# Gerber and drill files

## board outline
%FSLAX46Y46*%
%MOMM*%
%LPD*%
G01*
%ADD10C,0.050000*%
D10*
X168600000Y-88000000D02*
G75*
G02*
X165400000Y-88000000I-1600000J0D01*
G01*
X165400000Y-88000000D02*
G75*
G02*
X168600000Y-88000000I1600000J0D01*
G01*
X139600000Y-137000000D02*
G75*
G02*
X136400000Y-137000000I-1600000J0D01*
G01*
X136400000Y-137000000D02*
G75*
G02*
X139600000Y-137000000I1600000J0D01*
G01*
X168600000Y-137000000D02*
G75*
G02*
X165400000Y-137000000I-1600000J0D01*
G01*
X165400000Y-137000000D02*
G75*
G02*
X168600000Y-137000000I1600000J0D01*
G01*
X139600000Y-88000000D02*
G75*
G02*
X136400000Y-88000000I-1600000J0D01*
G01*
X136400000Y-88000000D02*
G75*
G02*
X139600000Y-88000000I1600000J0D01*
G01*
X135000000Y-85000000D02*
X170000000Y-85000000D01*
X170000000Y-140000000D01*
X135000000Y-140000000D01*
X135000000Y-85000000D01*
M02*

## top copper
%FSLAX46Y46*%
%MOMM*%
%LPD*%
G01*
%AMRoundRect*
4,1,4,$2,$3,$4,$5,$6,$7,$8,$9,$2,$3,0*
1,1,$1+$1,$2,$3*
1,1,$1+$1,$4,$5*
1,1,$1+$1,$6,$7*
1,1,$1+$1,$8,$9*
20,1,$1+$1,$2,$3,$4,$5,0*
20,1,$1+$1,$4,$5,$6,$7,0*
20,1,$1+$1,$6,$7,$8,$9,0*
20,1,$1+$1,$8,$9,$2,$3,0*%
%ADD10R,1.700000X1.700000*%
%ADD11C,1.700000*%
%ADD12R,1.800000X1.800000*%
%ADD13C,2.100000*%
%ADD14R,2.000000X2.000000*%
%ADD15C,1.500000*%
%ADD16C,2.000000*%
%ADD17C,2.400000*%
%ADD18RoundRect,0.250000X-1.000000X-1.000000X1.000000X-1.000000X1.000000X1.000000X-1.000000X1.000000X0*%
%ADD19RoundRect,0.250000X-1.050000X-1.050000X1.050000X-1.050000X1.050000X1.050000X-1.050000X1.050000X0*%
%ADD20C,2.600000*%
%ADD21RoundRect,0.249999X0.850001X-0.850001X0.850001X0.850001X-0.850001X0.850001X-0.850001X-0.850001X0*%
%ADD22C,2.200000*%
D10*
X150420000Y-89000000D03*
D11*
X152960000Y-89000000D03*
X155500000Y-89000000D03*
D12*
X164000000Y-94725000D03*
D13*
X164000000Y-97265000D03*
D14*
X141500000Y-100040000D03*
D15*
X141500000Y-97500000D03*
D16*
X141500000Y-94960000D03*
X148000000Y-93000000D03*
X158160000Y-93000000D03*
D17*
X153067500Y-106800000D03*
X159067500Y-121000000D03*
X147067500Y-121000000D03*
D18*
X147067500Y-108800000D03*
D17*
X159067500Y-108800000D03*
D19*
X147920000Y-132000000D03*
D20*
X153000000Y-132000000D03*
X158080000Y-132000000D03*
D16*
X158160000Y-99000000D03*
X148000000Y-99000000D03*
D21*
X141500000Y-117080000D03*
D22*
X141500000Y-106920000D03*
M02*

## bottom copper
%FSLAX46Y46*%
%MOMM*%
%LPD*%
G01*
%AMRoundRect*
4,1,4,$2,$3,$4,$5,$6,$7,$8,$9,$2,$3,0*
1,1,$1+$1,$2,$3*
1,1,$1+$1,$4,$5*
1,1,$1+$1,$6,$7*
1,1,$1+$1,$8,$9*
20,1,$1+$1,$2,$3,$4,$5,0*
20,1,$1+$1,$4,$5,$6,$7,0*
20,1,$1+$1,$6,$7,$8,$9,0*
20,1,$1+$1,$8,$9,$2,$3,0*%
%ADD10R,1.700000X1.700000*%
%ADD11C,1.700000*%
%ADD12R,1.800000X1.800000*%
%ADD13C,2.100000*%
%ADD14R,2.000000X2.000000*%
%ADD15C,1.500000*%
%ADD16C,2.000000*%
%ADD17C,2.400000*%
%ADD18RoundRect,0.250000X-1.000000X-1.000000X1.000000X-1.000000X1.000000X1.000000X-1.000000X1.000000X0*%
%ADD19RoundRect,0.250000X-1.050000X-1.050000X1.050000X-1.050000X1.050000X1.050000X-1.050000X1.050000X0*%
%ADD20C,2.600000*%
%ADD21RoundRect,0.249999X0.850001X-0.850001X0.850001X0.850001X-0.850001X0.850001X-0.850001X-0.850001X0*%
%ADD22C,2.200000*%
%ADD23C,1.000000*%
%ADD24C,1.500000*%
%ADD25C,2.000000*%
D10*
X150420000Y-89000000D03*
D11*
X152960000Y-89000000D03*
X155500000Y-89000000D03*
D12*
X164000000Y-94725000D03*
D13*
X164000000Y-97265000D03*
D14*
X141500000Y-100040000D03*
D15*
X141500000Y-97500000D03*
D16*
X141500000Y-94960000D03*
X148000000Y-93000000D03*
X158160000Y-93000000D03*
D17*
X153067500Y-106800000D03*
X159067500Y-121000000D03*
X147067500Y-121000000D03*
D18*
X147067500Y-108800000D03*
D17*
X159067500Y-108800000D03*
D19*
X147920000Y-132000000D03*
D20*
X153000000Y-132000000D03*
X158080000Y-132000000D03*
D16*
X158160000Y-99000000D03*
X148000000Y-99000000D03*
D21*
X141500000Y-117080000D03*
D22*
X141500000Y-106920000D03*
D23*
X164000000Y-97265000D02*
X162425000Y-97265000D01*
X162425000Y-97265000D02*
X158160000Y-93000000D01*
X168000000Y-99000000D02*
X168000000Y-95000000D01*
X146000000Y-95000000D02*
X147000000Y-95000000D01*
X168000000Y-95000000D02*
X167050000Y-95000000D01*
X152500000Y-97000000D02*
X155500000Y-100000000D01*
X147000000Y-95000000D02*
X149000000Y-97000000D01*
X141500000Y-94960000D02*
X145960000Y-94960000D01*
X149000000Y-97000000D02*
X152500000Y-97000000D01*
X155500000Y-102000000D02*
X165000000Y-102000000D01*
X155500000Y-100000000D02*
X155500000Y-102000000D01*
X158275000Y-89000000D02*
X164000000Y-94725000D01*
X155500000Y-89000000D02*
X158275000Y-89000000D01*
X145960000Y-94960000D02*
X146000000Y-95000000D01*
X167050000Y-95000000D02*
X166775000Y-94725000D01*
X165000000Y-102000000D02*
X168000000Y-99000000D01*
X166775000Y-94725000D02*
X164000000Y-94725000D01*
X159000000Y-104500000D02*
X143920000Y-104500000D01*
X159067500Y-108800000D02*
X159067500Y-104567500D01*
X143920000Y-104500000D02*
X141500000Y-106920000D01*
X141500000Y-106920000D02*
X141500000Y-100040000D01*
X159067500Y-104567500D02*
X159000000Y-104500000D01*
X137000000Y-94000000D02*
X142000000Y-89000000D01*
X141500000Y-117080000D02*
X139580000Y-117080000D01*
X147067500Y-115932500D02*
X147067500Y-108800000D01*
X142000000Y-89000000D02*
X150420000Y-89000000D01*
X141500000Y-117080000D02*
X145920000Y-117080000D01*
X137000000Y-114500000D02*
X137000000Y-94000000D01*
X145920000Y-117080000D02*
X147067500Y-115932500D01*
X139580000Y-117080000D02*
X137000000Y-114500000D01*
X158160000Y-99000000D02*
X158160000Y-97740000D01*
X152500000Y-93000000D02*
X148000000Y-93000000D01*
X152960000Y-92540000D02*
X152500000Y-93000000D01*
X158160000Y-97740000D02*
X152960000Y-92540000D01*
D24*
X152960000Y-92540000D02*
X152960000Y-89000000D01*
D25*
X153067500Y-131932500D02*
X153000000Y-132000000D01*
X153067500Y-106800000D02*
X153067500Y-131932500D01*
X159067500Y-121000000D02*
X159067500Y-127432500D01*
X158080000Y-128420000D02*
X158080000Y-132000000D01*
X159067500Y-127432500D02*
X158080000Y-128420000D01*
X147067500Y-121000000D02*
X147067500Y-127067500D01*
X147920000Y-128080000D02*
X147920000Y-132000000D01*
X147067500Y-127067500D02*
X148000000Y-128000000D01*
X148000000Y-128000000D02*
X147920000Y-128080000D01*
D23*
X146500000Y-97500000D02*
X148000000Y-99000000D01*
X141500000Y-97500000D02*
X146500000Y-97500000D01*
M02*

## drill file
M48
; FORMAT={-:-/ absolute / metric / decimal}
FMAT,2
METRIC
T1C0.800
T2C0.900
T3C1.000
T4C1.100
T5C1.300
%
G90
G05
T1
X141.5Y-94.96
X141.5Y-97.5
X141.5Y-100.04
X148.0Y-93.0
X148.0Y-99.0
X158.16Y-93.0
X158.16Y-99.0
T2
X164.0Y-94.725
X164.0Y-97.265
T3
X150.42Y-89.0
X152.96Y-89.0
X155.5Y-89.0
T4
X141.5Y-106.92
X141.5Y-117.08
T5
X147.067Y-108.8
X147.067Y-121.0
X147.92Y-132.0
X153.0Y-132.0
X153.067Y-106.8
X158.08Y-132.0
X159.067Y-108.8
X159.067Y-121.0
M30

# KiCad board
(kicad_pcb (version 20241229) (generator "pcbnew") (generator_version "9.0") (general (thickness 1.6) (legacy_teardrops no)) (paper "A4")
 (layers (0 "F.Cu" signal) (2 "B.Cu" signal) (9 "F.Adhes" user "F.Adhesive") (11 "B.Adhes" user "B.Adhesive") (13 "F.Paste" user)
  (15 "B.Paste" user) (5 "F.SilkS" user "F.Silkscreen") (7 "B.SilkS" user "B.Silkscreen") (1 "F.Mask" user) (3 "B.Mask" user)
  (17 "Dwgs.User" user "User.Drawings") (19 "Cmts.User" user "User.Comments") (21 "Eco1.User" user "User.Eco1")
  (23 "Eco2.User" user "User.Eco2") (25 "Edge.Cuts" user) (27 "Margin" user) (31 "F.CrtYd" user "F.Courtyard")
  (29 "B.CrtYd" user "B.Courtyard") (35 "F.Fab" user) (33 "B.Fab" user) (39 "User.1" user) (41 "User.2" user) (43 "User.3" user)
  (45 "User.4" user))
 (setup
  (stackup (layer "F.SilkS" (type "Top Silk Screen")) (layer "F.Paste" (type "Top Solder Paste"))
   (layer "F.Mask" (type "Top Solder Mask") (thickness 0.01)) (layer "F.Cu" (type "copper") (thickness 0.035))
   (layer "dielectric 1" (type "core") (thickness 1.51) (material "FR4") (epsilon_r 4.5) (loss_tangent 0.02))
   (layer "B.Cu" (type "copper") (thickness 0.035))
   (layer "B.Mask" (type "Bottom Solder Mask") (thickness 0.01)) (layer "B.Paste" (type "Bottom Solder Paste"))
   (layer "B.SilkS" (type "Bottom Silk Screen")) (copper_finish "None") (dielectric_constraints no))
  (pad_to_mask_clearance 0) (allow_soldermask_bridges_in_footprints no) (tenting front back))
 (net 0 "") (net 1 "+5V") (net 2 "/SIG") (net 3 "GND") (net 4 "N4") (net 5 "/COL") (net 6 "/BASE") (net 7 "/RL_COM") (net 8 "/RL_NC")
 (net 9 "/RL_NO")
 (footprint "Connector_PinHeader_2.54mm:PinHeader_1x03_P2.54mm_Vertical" (layer "F.Cu") (at 150.42 89 90)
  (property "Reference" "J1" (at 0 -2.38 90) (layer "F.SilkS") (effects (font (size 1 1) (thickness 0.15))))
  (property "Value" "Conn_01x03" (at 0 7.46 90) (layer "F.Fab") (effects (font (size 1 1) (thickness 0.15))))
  (pad "1" thru_hole rect (at 0 0 90) (size 1.7 1.7) (drill 1) (layers "*.Cu" "*.Mask") (remove_unused_layers no) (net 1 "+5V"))
  (pad "2" thru_hole circle (at 0 2.54 90) (size 1.7 1.7) (drill 1) (layers "*.Cu" "*.Mask") (remove_unused_layers no) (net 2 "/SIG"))
  (pad "3" thru_hole circle (at 0 5.08 90) (size 1.7 1.7) (drill 1) (layers "*.Cu" "*.Mask") (remove_unused_layers no) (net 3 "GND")))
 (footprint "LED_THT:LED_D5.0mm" (layer "F.Cu") (at 164 94.725 -90)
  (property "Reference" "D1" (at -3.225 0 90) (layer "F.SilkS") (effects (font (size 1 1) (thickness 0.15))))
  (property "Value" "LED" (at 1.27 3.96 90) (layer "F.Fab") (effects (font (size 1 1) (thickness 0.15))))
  (pad "1" thru_hole rect (at 0 0 270) (size 1.8 1.8) (drill 0.9) (layers "*.Cu" "*.Mask") (remove_unused_layers no) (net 3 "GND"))
  (pad "2" thru_hole circle (at 2.54 0 270) (size 2.1 2.1) (drill 0.9) (layers "*.Cu" "*.Mask") (remove_unused_layers no) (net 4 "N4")))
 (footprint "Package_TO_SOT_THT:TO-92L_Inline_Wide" (layer "F.Cu") (at 141.5 100.04 90)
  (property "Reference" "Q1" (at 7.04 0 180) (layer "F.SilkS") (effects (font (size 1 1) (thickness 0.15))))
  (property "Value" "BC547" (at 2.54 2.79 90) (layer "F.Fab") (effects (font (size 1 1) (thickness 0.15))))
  (pad "1" thru_hole rect (at 0 0 90) (size 2 2) (drill 0.8) (layers "*.Cu" "*.Mask") (remove_unused_layers no) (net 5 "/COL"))
  (pad "2" thru_hole circle (at 2.54 0 90) (size 1.5 1.5) (drill 0.8) (layers "*.Cu" "*.Mask") (remove_unused_layers no) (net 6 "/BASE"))
  (pad "3" thru_hole circle (at 5.08 0 90) (size 2 2) (drill 0.8) (layers "*.Cu" "*.Mask") (remove_unused_layers no) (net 3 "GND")))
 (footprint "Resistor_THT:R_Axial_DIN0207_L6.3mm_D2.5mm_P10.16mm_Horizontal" (layer "F.Cu") (at 148 93)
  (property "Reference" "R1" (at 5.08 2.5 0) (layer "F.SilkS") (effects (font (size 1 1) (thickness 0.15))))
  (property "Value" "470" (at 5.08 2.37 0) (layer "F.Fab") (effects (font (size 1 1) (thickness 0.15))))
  (pad "1" thru_hole circle (at 0 0) (size 2 2) (drill 0.8) (layers "*.Cu" "*.Mask") (remove_unused_layers no) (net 2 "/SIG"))
  (pad "2" thru_hole circle (at 10.16 0) (size 2 2) (drill 0.8) (layers "*.Cu" "*.Mask") (remove_unused_layers no) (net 4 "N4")))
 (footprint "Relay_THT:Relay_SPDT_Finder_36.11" (layer "F.Cu") (at 147.0675 108.8)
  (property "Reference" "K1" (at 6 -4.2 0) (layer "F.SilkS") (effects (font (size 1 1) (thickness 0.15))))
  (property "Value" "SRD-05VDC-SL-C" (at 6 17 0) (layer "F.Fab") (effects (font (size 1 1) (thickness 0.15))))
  (pad "11" thru_hole circle (at 6 -2) (size 2.4 2.4) (drill 1.3) (layers "*.Cu" "*.Mask") (remove_unused_layers no) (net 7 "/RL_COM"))
  (pad "12" thru_hole circle (at 12 12.2) (size 2.4 2.4) (drill 1.3) (layers "*.Cu" "*.Mask") (remove_unused_layers no) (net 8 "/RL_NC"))
  (pad "14" thru_hole circle (at 0 12.2) (size 2.4 2.4) (drill 1.3) (layers "*.Cu" "*.Mask") (remove_unused_layers no) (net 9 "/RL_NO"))
  (pad "A1" thru_hole roundrect (at 0 0) (size 2.5 2.5) (drill 1.3) (layers "*.Cu" "*.Mask") (remove_unused_layers no)
   (roundrect_rratio 0.1) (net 1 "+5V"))
  (pad "A2" thru_hole circle (at 12 0) (size 2.4 2.4) (drill 1.3) (layers "*.Cu" "*.Mask") (remove_unused_layers no) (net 5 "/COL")))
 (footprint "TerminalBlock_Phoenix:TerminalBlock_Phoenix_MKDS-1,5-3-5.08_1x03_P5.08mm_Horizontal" (layer "F.Cu") (at 147.92 132)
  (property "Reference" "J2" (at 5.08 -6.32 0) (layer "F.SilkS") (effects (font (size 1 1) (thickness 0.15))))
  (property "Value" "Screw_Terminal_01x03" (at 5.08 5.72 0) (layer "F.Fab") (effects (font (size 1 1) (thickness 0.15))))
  (pad "1" thru_hole roundrect (at 0 0) (size 2.6 2.6) (drill 1.3) (layers "*.Cu" "*.Mask") (remove_unused_layers no)
   (roundrect_rratio 0.096154) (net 9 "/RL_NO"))
  (pad "2" thru_hole circle (at 5.08 0) (size 2.6 2.6) (drill 1.3) (layers "*.Cu" "*.Mask") (remove_unused_layers no) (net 7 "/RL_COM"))
  (pad "3" thru_hole circle (at 10.16 0) (size 2.6 2.6) (drill 1.3) (layers "*.Cu" "*.Mask") (remove_unused_layers no) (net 8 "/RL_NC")))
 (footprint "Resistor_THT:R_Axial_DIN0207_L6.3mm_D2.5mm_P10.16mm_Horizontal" (layer "F.Cu") (at 158.16 99 180)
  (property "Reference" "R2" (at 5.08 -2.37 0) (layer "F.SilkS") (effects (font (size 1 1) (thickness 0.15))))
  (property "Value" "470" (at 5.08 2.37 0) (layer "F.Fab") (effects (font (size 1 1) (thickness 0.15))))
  (pad "1" thru_hole circle (at 0 0 180) (size 2 2) (drill 0.8) (layers "*.Cu" "*.Mask") (remove_unused_layers no) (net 2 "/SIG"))
  (pad "2" thru_hole circle (at 10.16 0 180) (size 2 2) (drill 0.8) (layers "*.Cu" "*.Mask") (remove_unused_layers no) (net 6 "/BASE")))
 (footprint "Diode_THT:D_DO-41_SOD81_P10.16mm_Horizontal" (layer "F.Cu") (at 141.5 117.08 90)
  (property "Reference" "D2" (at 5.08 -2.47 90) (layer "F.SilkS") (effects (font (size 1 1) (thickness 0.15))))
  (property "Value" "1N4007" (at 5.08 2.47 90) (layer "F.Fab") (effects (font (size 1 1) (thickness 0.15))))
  (pad "1" thru_hole roundrect (at 0 0 90) (size 2.2 2.2) (drill 1.1) (layers "*.Cu" "*.Mask") (remove_unused_layers no)
   (roundrect_rratio 0.113636) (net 1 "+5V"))
  (pad "2" thru_hole circle (at 10.16 0 90) (size 2.2 2.2) (drill 1.1) (layers "*.Cu" "*.Mask") (remove_unused_layers no) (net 5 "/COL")))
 (gr_circle (center 167 88) (end 168.6 88) (stroke (width 0.05) (type default)) (fill no) (locked yes) (layer "Edge.Cuts"))
 (gr_circle (center 138 137) (end 139.6 137) (stroke (width 0.05) (type default)) (fill no) (locked yes) (layer "Edge.Cuts"))
 (gr_circle (center 167 137) (end 168.6 137) (stroke (width 0.05) (type default)) (fill no) (locked yes) (layer "Edge.Cuts"))
 (gr_circle (center 138 88) (end 139.6 88) (stroke (width 0.05) (type default)) (fill no) (locked yes) (layer "Edge.Cuts"))
 (gr_rect (start 135 85) (end 170 140) (stroke (width 0.05) (type default)) (fill no) (locked yes) (layer "Edge.Cuts"))
 (segment (start 164 97.265) (end 162.425 97.265) (width 1) (layer "B.Cu") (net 4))
 (segment (start 162.425 97.265) (end 158.16 93) (width 1) (layer "B.Cu") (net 4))
 (segment (start 168 99) (end 168 95) (width 1) (layer "B.Cu") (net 3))
 (segment (start 146 95) (end 147 95) (width 1) (layer "B.Cu") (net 3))
 (segment (start 168 95) (end 167.05 95) (width 1) (layer "B.Cu") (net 3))
 (segment (start 152.5 97) (end 155.5 100) (width 1) (layer "B.Cu") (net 3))
 (segment (start 147 95) (end 149 97) (width 1) (layer "B.Cu") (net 3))
 (segment (start 141.5 94.96) (end 145.96 94.96) (width 1) (layer "B.Cu") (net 3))
 (segment (start 149 97) (end 152.5 97) (width 1) (layer "B.Cu") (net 3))
 (segment (start 155.5 102) (end 165 102) (width 1) (layer "B.Cu") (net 3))
 (segment (start 155.5 100) (end 155.5 102) (width 1) (layer "B.Cu") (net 3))
 (segment (start 158.275 89) (end 164 94.725) (width 1) (layer "B.Cu") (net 3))
 (segment (start 155.5 89) (end 158.275 89) (width 1) (layer "B.Cu") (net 3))
 (segment (start 145.96 94.96) (end 146 95) (width 1) (layer "B.Cu") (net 3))
 (segment (start 167.05 95) (end 166.775 94.725) (width 1) (layer "B.Cu") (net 3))
 (segment (start 165 102) (end 168 99) (width 1) (layer "B.Cu") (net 3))
 (segment (start 166.775 94.725) (end 164 94.725) (width 1) (layer "B.Cu") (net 3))
 (segment (start 159 104.5) (end 143.92 104.5) (width 1) (layer "B.Cu") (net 5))
 (segment (start 159.0675 108.8) (end 159.0675 104.5675) (width 1) (layer "B.Cu") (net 5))
 (segment (start 143.92 104.5) (end 141.5 106.92) (width 1) (layer "B.Cu") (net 5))
 (segment (start 141.5 106.92) (end 141.5 100.04) (width 1) (layer "B.Cu") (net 5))
 (segment (start 159.0675 104.5675) (end 159 104.5) (width 1) (layer "B.Cu") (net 5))
 (segment (start 137 94) (end 142 89) (width 1) (layer "B.Cu") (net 1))
 (segment (start 141.5 117.08) (end 139.58 117.08) (width 1) (layer "B.Cu") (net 1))
 (segment (start 147.0675 115.9325) (end 147.0675 108.8) (width 1) (layer "B.Cu") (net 1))
 (segment (start 142 89) (end 150.42 89) (width 1) (layer "B.Cu") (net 1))
 (segment (start 141.5 117.08) (end 145.92 117.08) (width 1) (layer "B.Cu") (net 1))
 (segment (start 137 114.5) (end 137 94) (width 1) (layer "B.Cu") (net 1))
 (segment (start 145.92 117.08) (end 147.0675 115.9325) (width 1) (layer "B.Cu") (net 1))
 (segment (start 139.58 117.08) (end 137 114.5) (width 1) (layer "B.Cu") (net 1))
 (segment (start 158.16 99) (end 158.16 97.74) (width 1) (layer "B.Cu") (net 2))
 (segment (start 152.5 93) (end 148 93) (width 1) (layer "B.Cu") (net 2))
 (segment (start 152.96 92.54) (end 152.5 93) (width 1) (layer "B.Cu") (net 2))
 (segment (start 158.16 97.74) (end 152.96 92.54) (width 1) (layer "B.Cu") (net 2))
 (segment (start 152.96 92.54) (end 152.96 89) (width 1.5) (layer "B.Cu") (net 2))
 (segment (start 153.0675 131.9325) (end 153 132) (width 2) (layer "B.Cu") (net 7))
 (segment (start 153.0675 106.8) (end 153.0675 131.9325) (width 2) (layer "B.Cu") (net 7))
 (segment (start 159.0675 121) (end 159.0675 127.4325) (width 2) (layer "B.Cu") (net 8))
 (segment (start 158.08 128.42) (end 158.08 132) (width 2) (layer "B.Cu") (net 8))
 (segment (start 159.0675 127.4325) (end 158.08 128.42) (width 2) (layer "B.Cu") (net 8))
 (segment (start 147.0675 121) (end 147.0675 127.0675) (width 2) (layer "B.Cu") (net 9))
 (segment (start 147.92 128.08) (end 147.92 132) (width 2) (layer "B.Cu") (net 9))
 (segment (start 147.0675 127.0675) (end 148 128) (width 2) (layer "B.Cu") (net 9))
 (segment (start 148 128) (end 147.92 128.08) (width 2) (layer "B.Cu") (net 9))
 (segment (start 146.5 97.5) (end 148 99) (width 1) (layer "B.Cu") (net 6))
 (segment (start 141.5 97.5) (end 146.5 97.5) (width 1) (layer "B.Cu") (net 6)))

